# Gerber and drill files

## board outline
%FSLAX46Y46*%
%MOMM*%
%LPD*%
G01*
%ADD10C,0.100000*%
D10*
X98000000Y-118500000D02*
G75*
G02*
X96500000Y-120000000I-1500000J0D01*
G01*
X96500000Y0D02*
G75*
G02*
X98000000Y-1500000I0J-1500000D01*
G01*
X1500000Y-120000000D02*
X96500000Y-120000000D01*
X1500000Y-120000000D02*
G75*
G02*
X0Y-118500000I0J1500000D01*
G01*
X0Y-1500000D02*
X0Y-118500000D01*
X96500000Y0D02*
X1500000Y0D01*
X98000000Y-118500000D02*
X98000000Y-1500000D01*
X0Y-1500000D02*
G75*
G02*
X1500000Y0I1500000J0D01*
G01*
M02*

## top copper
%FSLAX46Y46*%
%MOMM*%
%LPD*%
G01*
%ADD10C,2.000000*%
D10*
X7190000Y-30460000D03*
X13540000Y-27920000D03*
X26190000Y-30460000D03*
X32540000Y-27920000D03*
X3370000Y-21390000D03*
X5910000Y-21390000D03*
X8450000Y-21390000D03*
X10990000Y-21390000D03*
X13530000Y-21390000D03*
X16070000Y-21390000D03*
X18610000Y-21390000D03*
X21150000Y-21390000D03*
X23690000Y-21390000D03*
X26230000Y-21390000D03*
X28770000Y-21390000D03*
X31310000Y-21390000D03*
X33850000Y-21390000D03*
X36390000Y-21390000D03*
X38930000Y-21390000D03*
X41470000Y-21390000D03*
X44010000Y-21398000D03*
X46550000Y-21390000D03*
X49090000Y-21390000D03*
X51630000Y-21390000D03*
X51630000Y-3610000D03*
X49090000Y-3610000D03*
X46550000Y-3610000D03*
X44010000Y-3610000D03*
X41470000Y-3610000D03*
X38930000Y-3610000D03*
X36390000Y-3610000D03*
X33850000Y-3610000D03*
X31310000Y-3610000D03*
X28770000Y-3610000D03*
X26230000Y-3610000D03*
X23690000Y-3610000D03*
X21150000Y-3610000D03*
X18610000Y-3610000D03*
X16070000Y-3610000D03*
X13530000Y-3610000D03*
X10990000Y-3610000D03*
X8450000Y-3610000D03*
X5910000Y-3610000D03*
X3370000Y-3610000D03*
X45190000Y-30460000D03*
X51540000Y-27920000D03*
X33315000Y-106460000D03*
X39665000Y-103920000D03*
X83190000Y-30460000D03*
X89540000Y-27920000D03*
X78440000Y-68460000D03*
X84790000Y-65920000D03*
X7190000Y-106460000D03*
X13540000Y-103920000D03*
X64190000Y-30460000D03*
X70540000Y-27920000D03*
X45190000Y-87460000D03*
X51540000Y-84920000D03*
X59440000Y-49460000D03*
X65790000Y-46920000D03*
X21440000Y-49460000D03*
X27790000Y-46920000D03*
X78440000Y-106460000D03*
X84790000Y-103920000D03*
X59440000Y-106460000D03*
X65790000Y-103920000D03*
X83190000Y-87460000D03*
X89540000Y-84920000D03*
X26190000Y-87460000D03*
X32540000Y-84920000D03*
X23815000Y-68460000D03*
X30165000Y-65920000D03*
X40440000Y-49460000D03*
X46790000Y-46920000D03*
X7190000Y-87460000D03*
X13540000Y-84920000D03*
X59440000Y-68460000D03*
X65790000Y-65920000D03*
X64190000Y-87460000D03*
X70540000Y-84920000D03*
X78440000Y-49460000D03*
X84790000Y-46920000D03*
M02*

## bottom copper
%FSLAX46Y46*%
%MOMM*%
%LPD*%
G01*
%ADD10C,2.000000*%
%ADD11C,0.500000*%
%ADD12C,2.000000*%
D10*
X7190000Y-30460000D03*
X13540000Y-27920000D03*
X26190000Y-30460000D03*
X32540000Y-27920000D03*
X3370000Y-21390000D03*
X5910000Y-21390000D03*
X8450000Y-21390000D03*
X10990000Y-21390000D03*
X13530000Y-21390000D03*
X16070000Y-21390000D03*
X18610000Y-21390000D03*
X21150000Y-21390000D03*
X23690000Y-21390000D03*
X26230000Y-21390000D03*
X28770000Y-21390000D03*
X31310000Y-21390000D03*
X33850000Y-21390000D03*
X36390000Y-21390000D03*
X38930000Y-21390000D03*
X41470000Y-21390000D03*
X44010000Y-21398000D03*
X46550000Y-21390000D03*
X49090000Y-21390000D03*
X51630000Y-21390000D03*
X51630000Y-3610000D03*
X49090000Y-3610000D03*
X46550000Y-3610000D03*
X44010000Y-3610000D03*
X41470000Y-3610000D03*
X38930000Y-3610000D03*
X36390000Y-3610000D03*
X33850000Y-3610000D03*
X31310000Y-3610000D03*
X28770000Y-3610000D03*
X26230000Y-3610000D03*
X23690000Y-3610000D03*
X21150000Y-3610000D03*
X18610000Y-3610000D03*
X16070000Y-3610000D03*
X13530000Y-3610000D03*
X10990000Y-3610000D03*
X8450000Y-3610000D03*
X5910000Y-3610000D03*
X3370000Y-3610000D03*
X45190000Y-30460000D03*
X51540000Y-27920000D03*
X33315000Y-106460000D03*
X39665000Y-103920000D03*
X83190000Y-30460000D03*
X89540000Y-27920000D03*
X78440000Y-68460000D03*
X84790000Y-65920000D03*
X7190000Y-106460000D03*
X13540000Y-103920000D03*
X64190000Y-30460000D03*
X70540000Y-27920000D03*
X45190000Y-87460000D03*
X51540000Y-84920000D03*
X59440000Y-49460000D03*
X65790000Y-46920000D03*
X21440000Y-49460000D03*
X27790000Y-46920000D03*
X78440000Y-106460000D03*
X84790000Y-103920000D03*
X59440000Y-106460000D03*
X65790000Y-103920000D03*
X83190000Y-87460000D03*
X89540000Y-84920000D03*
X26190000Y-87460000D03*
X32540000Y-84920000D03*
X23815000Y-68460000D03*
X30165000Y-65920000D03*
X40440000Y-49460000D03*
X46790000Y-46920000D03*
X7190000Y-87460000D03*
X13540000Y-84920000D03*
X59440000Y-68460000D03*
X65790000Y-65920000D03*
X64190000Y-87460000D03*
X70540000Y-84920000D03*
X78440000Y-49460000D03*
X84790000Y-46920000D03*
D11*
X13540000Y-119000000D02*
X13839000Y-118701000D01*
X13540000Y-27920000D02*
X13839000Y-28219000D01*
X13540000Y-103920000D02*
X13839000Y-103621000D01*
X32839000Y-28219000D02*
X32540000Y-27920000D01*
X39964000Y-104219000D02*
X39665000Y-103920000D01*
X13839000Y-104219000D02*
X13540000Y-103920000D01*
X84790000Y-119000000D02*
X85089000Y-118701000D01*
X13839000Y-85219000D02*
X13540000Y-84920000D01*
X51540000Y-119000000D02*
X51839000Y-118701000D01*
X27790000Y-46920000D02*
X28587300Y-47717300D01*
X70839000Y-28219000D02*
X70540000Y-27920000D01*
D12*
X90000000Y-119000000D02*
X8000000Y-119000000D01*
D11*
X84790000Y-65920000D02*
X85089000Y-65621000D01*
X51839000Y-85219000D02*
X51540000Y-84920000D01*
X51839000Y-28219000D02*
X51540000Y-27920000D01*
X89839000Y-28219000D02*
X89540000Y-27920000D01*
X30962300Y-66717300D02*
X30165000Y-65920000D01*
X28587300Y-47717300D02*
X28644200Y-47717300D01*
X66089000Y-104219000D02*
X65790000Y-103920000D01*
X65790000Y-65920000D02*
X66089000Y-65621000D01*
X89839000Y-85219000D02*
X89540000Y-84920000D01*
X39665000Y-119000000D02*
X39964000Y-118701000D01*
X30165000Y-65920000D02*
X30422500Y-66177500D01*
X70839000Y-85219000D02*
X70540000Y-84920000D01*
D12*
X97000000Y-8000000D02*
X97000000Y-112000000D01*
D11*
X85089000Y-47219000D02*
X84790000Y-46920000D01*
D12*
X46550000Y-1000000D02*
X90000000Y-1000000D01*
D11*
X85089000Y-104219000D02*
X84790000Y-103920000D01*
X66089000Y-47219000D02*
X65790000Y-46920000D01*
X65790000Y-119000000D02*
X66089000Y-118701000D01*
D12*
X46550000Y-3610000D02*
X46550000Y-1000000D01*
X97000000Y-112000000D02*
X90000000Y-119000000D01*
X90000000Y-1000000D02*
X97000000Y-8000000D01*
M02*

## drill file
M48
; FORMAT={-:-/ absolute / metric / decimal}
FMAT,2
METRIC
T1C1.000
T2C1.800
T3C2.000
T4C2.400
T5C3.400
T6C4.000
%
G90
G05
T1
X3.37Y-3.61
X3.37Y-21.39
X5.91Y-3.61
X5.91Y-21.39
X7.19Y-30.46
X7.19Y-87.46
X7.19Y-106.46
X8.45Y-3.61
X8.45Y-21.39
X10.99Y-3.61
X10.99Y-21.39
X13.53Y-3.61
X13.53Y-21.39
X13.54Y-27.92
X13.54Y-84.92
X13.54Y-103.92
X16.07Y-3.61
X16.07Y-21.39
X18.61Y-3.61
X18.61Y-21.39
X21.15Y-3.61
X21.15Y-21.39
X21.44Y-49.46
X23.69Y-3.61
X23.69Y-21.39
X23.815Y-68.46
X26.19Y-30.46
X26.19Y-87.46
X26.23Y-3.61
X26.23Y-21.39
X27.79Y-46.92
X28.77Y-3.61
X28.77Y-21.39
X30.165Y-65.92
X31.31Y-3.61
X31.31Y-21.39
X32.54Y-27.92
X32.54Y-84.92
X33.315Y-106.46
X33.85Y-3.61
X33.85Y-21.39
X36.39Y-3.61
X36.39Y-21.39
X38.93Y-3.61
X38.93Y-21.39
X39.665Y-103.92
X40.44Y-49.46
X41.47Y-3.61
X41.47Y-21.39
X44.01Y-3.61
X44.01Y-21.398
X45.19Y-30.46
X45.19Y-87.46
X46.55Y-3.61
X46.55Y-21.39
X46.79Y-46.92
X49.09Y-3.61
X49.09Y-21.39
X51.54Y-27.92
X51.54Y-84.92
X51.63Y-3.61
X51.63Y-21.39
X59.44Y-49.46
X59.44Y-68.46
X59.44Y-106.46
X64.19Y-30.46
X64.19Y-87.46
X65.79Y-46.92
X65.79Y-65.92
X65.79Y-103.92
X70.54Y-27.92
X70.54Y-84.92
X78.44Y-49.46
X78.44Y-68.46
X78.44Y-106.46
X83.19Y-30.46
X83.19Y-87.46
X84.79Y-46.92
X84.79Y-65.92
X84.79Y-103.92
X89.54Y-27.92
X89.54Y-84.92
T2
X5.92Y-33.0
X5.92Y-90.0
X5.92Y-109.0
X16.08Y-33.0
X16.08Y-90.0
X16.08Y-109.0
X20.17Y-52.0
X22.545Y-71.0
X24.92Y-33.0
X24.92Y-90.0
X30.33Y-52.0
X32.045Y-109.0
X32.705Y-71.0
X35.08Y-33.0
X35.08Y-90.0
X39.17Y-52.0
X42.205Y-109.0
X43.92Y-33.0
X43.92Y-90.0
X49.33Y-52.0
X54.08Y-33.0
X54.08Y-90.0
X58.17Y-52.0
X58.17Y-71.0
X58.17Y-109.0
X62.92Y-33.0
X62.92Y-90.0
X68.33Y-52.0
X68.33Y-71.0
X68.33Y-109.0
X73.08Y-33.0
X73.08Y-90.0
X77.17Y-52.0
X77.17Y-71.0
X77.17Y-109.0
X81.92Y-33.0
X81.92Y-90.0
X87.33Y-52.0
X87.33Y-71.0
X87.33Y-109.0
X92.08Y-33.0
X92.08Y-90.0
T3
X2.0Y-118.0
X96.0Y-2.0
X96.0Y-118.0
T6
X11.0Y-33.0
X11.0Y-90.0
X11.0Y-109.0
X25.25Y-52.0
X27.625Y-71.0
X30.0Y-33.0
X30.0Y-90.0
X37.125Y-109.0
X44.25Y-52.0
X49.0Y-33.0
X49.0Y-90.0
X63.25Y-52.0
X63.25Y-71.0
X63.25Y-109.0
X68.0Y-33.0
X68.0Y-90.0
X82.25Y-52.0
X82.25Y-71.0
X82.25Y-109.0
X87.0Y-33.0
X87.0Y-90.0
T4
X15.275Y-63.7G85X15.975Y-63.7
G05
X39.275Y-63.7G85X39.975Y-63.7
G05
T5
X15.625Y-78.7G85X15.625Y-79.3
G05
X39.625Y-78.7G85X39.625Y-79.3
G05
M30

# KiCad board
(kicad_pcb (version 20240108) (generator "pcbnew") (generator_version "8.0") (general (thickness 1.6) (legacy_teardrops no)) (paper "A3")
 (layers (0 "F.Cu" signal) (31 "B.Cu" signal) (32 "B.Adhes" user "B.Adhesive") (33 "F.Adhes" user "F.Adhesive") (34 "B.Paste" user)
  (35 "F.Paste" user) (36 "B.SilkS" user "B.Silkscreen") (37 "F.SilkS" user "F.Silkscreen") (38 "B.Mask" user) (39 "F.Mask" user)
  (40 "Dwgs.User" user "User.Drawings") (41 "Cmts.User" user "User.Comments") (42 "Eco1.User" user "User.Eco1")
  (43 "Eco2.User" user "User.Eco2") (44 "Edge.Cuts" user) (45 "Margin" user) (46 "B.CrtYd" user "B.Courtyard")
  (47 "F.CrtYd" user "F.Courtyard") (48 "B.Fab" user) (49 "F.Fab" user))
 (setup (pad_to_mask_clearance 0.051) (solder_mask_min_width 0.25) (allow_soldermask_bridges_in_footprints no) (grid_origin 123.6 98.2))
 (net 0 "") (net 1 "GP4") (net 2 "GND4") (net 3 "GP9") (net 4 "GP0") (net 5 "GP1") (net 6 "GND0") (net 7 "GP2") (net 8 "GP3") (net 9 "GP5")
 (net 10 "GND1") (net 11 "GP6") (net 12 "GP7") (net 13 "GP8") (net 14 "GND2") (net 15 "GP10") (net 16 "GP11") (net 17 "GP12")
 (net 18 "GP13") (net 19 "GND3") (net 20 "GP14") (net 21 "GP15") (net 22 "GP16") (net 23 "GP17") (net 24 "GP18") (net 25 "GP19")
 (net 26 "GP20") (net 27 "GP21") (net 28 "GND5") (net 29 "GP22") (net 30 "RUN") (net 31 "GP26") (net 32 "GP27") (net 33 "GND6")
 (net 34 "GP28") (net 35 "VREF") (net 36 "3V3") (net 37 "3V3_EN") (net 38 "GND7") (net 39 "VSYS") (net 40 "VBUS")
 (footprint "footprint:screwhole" (layer "F.Cu") (at 96 2)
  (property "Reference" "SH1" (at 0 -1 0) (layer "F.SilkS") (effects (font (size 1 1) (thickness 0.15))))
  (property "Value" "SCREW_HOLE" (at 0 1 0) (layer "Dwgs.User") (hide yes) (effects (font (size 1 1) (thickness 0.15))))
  (pad "" np_thru_hole circle (at 0 0) (size 2 2) (drill 2) (layers "*.Cu" "*.Mask")))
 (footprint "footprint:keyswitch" (layer "F.Cu") (at 11 33)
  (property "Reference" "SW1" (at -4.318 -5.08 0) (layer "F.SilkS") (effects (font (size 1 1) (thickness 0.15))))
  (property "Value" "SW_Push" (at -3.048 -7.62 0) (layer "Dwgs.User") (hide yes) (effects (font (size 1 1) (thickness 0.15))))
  (pad "" np_thru_hole circle (at -5.08 0) (size 1.8 1.8) (drill 1.8) (layers "*.Cu" "*.Mask"))
  (pad "" np_thru_hole circle (at 0 0) (size 4 4) (drill 4) (layers "*.Cu" "*.Mask"))
  (pad "" np_thru_hole circle (at 5.08 0) (size 1.8 1.8) (drill 1.8) (layers "*.Cu" "*.Mask"))
  (pad "1" thru_hole circle (at -3.81 -2.54) (size 2 2) (drill 1) (layers "*.Cu" "*.Mask") (remove_unused_layers no) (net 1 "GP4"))
  (pad "2" thru_hole circle (at 2.54 -5.08) (size 2 2) (drill 1) (layers "*.Cu" "*.Mask") (remove_unused_layers no) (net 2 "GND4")))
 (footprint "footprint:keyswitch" (layer "F.Cu") (at 30 33)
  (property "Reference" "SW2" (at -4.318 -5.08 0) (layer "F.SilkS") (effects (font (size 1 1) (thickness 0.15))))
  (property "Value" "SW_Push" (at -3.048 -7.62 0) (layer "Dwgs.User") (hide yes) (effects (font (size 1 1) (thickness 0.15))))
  (pad "" np_thru_hole circle (at -5.08 0) (size 1.8 1.8) (drill 1.8) (layers "*.Cu" "*.Mask"))
  (pad "" np_thru_hole circle (at 0 0) (size 4 4) (drill 4) (layers "*.Cu" "*.Mask"))
  (pad "" np_thru_hole circle (at 5.08 0) (size 1.8 1.8) (drill 1.8) (layers "*.Cu" "*.Mask"))
  (pad "1" thru_hole circle (at -3.81 -2.54) (size 2 2) (drill 1) (layers "*.Cu" "*.Mask") (remove_unused_layers no) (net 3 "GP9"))
  (pad "2" thru_hole circle (at 2.54 -5.08) (size 2 2) (drill 1) (layers "*.Cu" "*.Mask") (remove_unused_layers no) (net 2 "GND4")))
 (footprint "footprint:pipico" (layer "F.Cu") (at 27.5 12.5)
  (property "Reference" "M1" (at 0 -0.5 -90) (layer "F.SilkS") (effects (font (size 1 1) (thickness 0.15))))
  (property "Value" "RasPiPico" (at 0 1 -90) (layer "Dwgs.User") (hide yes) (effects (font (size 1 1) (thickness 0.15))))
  (pad "1" thru_hole circle (at -24.13 8.89 270) (size 2 2) (drill 1) (layers "*.Cu" "*.Mask") (remove_unused_layers no) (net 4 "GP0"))
  (pad "2" thru_hole circle (at -21.59 8.89 270) (size 2 2) (drill 1) (layers "*.Cu" "*.Mask") (remove_unused_layers no) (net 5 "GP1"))
  (pad "3" thru_hole circle (at -19.05 8.89 270) (size 2 2) (drill 1) (layers "*.Cu" "*.Mask") (remove_unused_layers no) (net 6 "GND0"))
  (pad "4" thru_hole circle (at -16.51 8.89 270) (size 2 2) (drill 1) (layers "*.Cu" "*.Mask") (remove_unused_layers no) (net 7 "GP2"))
  (pad "5" thru_hole circle (at -13.97 8.89 270) (size 2 2) (drill 1) (layers "*.Cu" "*.Mask") (remove_unused_layers no) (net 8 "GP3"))
  (pad "6" thru_hole circle (at -11.43 8.89 270) (size 2 2) (drill 1) (layers "*.Cu" "*.Mask") (remove_unused_layers no) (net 1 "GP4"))
  (pad "7" thru_hole circle (at -8.89 8.89 270) (size 2 2) (drill 1) (layers "*.Cu" "*.Mask") (remove_unused_layers no) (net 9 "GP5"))
  (pad "8" thru_hole circle (at -6.35 8.89 270) (size 2 2) (drill 1) (layers "*.Cu" "*.Mask") (remove_unused_layers no) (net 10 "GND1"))
  (pad "9" thru_hole circle (at -3.81 8.89 270) (size 2 2) (drill 1) (layers "*.Cu" "*.Mask") (remove_unused_layers no) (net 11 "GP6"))
  (pad "10" thru_hole circle (at -1.27 8.89 270) (size 2 2) (drill 1) (layers "*.Cu" "*.Mask") (remove_unused_layers no) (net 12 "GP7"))
  (pad "11" thru_hole circle (at 1.27 8.89 270) (size 2 2) (drill 1) (layers "*.Cu" "*.Mask") (remove_unused_layers no) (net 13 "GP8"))
  (pad "12" thru_hole circle (at 3.81 8.89 270) (size 2 2) (drill 1) (layers "*.Cu" "*.Mask") (remove_unused_layers no) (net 3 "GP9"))
  (pad "13" thru_hole circle (at 6.35 8.89 270) (size 2 2) (drill 1) (layers "*.Cu" "*.Mask") (remove_unused_layers no) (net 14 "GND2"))
  (pad "14" thru_hole circle (at 8.89 8.89 270) (size 2 2) (drill 1) (layers "*.Cu" "*.Mask") (remove_unused_layers no) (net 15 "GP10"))
  (pad "15" thru_hole circle (at 11.43 8.89 270) (size 2 2) (drill 1) (layers "*.Cu" "*.Mask") (remove_unused_layers no) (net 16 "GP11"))
  (pad "16" thru_hole circle (at 13.97 8.89 270) (size 2 2) (drill 1) (layers "*.Cu" "*.Mask") (remove_unused_layers no) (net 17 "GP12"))
  (pad "17" thru_hole circle (at 16.51 8.898 270) (size 2 2) (drill 1) (layers "*.Cu" "*.Mask") (remove_unused_layers no) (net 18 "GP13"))
  (pad "18" thru_hole circle (at 19.05 8.89 270) (size 2 2) (drill 1) (layers "*.Cu" "*.Mask") (remove_unused_layers no) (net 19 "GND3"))
  (pad "19" thru_hole circle (at 21.59 8.89 270) (size 2 2) (drill 1) (layers "*.Cu" "*.Mask") (remove_unused_layers no) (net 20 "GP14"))
  (pad "20" thru_hole circle (at 24.13 8.89 270) (size 2 2) (drill 1) (layers "*.Cu" "*.Mask") (remove_unused_layers no) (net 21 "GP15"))
  (pad "21" thru_hole circle (at 24.13 -8.89 270) (size 2 2) (drill 1) (layers "*.Cu" "*.Mask") (remove_unused_layers no) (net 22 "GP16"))
  (pad "22" thru_hole circle (at 21.59 -8.89 270) (size 2 2) (drill 1) (layers "*.Cu" "*.Mask") (remove_unused_layers no) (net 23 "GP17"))
  (pad "23" thru_hole circle (at 19.05 -8.89 270) (size 2 2) (drill 1) (layers "*.Cu" "*.Mask") (remove_unused_layers no) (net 2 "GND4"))
  (pad "24" thru_hole circle (at 16.51 -8.89 270) (size 2 2) (drill 1) (layers "*.Cu" "*.Mask") (remove_unused_layers no) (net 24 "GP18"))
  (pad "25" thru_hole circle (at 13.97 -8.89 270) (size 2 2) (drill 1) (layers "*.Cu" "*.Mask") (remove_unused_layers no) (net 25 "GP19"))
  (pad "26" thru_hole circle (at 11.43 -8.89 270) (size 2 2) (drill 1) (layers "*.Cu" "*.Mask") (remove_unused_layers no) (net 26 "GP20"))
  (pad "27" thru_hole circle (at 8.89 -8.89 270) (size 2 2) (drill 1) (layers "*.Cu" "*.Mask") (remove_unused_layers no) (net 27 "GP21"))
  (pad "28" thru_hole circle (at 6.35 -8.89 270) (size 2 2) (drill 1) (layers "*.Cu" "*.Mask") (remove_unused_layers no) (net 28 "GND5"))
  (pad "29" thru_hole circle (at 3.81 -8.89 270) (size 2 2) (drill 1) (layers "*.Cu" "*.Mask") (remove_unused_layers no) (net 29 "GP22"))
  (pad "30" thru_hole circle (at 1.27 -8.89 270) (size 2 2) (drill 1) (layers "*.Cu" "*.Mask") (remove_unused_layers no) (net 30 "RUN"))
  (pad "31" thru_hole circle (at -1.27 -8.89 270) (size 2 2) (drill 1) (layers "*.Cu" "*.Mask") (remove_unused_layers no) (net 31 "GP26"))
  (pad "32" thru_hole circle (at -3.81 -8.89 270) (size 2 2) (drill 1) (layers "*.Cu" "*.Mask") (remove_unused_layers no) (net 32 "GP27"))
  (pad "33" thru_hole circle (at -6.35 -8.89 270) (size 2 2) (drill 1) (layers "*.Cu" "*.Mask") (remove_unused_layers no) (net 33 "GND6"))
  (pad "34" thru_hole circle (at -8.89 -8.89 270) (size 2 2) (drill 1) (layers "*.Cu" "*.Mask") (remove_unused_layers no) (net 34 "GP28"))
  (pad "35" thru_hole circle (at -11.43 -8.89 270) (size 2 2) (drill 1) (layers "*.Cu" "*.Mask") (remove_unused_layers no) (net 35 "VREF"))
  (pad "36" thru_hole circle (at -13.97 -8.89 270) (size 2 2) (drill 1) (layers "*.Cu" "*.Mask") (remove_unused_layers no) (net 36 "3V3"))
  (pad "37" thru_hole circle (at -16.51 -8.89 270) (size 2 2) (drill 1) (layers "*.Cu" "*.Mask") (remove_unused_layers no) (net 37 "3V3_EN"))
  (pad "38" thru_hole circle (at -19.05 -8.89 270) (size 2 2) (drill 1) (layers "*.Cu" "*.Mask") (remove_unused_layers no) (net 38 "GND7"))
  (pad "39" thru_hole circle (at -21.59 -8.89 270) (size 2 2) (drill 1) (layers "*.Cu" "*.Mask") (remove_unused_layers no) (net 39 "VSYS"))
  (pad "40" thru_hole circle (at -24.13 -8.89 270) (size 2 2) (drill 1) (layers "*.Cu" "*.Mask") (remove_unused_layers no) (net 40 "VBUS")))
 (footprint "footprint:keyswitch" (layer "F.Cu") (at 49 33)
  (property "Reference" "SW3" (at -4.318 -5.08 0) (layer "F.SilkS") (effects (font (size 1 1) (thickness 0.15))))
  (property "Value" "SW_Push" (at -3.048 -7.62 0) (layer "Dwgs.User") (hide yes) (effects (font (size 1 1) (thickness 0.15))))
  (pad "" np_thru_hole circle (at -5.08 0) (size 1.8 1.8) (drill 1.8) (layers "*.Cu" "*.Mask"))
  (pad "" np_thru_hole circle (at 0 0) (size 4 4) (drill 4) (layers "*.Cu" "*.Mask"))
  (pad "" np_thru_hole circle (at 5.08 0) (size 1.8 1.8) (drill 1.8) (layers "*.Cu" "*.Mask"))
  (pad "1" thru_hole circle (at -3.81 -2.54) (size 2 2) (drill 1) (layers "*.Cu" "*.Mask") (remove_unused_layers no) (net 20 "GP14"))
  (pad "2" thru_hole circle (at 2.54 -5.08) (size 2 2) (drill 1) (layers "*.Cu" "*.Mask") (remove_unused_layers no) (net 2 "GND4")))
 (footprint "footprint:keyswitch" (layer "F.Cu") (at 37.125 109)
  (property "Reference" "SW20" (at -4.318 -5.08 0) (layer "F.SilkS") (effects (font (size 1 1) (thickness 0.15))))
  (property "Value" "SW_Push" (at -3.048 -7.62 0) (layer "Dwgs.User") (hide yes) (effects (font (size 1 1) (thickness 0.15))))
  (pad "" np_thru_hole circle (at -5.08 0) (size 1.8 1.8) (drill 1.8) (layers "*.Cu" "*.Mask"))
  (pad "" np_thru_hole circle (at 0 0) (size 4 4) (drill 4) (layers "*.Cu" "*.Mask"))
  (pad "" np_thru_hole circle (at 5.08 0) (size 1.8 1.8) (drill 1.8) (layers "*.Cu" "*.Mask"))
  (pad "1" thru_hole circle (at -3.81 -2.54) (size 2 2) (drill 1) (layers "*.Cu" "*.Mask") (remove_unused_layers no) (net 9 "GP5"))
  (pad "2" thru_hole circle (at 2.54 -5.08) (size 2 2) (drill 1) (layers "*.Cu" "*.Mask") (remove_unused_layers no) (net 2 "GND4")))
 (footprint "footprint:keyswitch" (layer "F.Cu") (at 87 33)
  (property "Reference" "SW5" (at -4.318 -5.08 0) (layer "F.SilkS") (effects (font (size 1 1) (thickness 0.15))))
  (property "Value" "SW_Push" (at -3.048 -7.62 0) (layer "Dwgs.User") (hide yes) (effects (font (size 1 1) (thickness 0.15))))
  (pad "" np_thru_hole circle (at -5.08 0) (size 1.8 1.8) (drill 1.8) (layers "*.Cu" "*.Mask"))
  (pad "" np_thru_hole circle (at 0 0) (size 4 4) (drill 4) (layers "*.Cu" "*.Mask"))
  (pad "" np_thru_hole circle (at 5.08 0) (size 1.8 1.8) (drill 1.8) (layers "*.Cu" "*.Mask"))
  (pad "1" thru_hole circle (at -3.81 -2.54) (size 2 2) (drill 1) (layers "*.Cu" "*.Mask") (remove_unused_layers no) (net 22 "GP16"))
  (pad "2" thru_hole circle (at 2.54 -5.08) (size 2 2) (drill 1) (layers "*.Cu" "*.Mask") (remove_unused_layers no) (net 2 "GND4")))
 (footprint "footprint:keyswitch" (layer "F.Cu") (at 82.25 71)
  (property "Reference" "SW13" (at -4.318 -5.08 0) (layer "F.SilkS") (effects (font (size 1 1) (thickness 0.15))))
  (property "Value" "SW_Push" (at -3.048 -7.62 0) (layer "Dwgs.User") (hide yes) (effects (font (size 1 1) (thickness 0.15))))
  (pad "" np_thru_hole circle (at -5.08 0) (size 1.8 1.8) (drill 1.8) (layers "*.Cu" "*.Mask"))
  (pad "" np_thru_hole circle (at 0 0) (size 4 4) (drill 4) (layers "*.Cu" "*.Mask"))
  (pad "" np_thru_hole circle (at 5.08 0) (size 1.8 1.8) (drill 1.8) (layers "*.Cu" "*.Mask"))
  (pad "1" thru_hole circle (at -3.81 -2.54) (size 2 2) (drill 1) (layers "*.Cu" "*.Mask") (remove_unused_layers no) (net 24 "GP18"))
  (pad "2" thru_hole circle (at 2.54 -5.08) (size 2 2) (drill 1) (layers "*.Cu" "*.Mask") (remove_unused_layers no) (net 2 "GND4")))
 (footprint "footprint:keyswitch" (layer "F.Cu") (at 11 109)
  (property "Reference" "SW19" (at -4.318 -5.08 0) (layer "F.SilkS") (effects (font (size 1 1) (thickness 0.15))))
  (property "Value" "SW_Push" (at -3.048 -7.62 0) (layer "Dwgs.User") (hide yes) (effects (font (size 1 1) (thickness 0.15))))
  (pad "" np_thru_hole circle (at -5.08 0) (size 1.8 1.8) (drill 1.8) (layers "*.Cu" "*.Mask"))
  (pad "" np_thru_hole circle (at 0 0) (size 4 4) (drill 4) (layers "*.Cu" "*.Mask"))
  (pad "" np_thru_hole circle (at 5.08 0) (size 1.8 1.8) (drill 1.8) (layers "*.Cu" "*.Mask"))
  (pad "1" thru_hole circle (at -3.81 -2.54) (size 2 2) (drill 1) (layers "*.Cu" "*.Mask") (remove_unused_layers no) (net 4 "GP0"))
  (pad "2" thru_hole circle (at 2.54 -5.08) (size 2 2) (drill 1) (layers "*.Cu" "*.Mask") (remove_unused_layers no) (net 2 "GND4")))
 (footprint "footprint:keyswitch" (layer "F.Cu") (at 68 33)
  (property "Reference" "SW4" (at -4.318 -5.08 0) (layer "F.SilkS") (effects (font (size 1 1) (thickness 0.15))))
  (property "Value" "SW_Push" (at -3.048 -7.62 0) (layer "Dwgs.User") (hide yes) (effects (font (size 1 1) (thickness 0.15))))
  (pad "" np_thru_hole circle (at -5.08 0) (size 1.8 1.8) (drill 1.8) (layers "*.Cu" "*.Mask"))
  (pad "" np_thru_hole circle (at 0 0) (size 4 4) (drill 4) (layers "*.Cu" "*.Mask"))
  (pad "" np_thru_hole circle (at 5.08 0) (size 1.8 1.8) (drill 1.8) (layers "*.Cu" "*.Mask"))
  (pad "1" thru_hole circle (at -3.81 -2.54) (size 2 2) (drill 1) (layers "*.Cu" "*.Mask") (remove_unused_layers no) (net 27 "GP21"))
  (pad "2" thru_hole circle (at 2.54 -5.08) (size 2 2) (drill 1) (layers "*.Cu" "*.Mask") (remove_unused_layers no) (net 2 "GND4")))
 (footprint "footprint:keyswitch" (layer "F.Cu") (at 49 90)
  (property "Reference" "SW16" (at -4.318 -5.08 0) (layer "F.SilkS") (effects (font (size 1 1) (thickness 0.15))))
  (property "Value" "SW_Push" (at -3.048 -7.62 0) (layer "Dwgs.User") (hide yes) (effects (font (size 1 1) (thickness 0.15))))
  (pad "" np_thru_hole circle (at -5.08 0) (size 1.8 1.8) (drill 1.8) (layers "*.Cu" "*.Mask"))
  (pad "" np_thru_hole circle (at 0 0) (size 4 4) (drill 4) (layers "*.Cu" "*.Mask"))
  (pad "" np_thru_hole circle (at 5.08 0) (size 1.8 1.8) (drill 1.8) (layers "*.Cu" "*.Mask"))
  (pad "1" thru_hole circle (at -3.81 -2.54) (size 2 2) (drill 1) (layers "*.Cu" "*.Mask") (remove_unused_layers no) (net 16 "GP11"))
  (pad "2" thru_hole circle (at 2.54 -5.08) (size 2 2) (drill 1) (layers "*.Cu" "*.Mask") (remove_unused_layers no) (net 2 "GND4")))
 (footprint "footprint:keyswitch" (layer "F.Cu") (at 63.25 52)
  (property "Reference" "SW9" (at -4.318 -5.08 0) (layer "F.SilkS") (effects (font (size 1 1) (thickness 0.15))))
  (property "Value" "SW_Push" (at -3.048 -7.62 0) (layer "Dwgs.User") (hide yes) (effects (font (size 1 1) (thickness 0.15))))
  (pad "" np_thru_hole circle (at -5.08 0) (size 1.8 1.8) (drill 1.8) (layers "*.Cu" "*.Mask"))
  (pad "" np_thru_hole circle (at 0 0) (size 4 4) (drill 4) (layers "*.Cu" "*.Mask"))
  (pad "" np_thru_hole circle (at 5.08 0) (size 1.8 1.8) (drill 1.8) (layers "*.Cu" "*.Mask"))
  (pad "1" thru_hole circle (at -3.81 -2.54) (size 2 2) (drill 1) (layers "*.Cu" "*.Mask") (remove_unused_layers no) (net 29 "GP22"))
  (pad "2" thru_hole circle (at 2.54 -5.08) (size 2 2) (drill 1) (layers "*.Cu" "*.Mask") (remove_unused_layers no) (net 2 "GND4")))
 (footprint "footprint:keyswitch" (layer "F.Cu") (at 25.25 52)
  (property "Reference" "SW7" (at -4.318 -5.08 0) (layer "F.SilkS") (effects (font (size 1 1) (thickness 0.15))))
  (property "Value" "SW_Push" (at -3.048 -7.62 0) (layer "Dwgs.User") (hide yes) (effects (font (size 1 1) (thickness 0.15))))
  (pad "" np_thru_hole circle (at -5.08 0) (size 1.8 1.8) (drill 1.8) (layers "*.Cu" "*.Mask"))
  (pad "" np_thru_hole circle (at 0 0) (size 4 4) (drill 4) (layers "*.Cu" "*.Mask"))
  (pad "" np_thru_hole circle (at 5.08 0) (size 1.8 1.8) (drill 1.8) (layers "*.Cu" "*.Mask"))
  (pad "1" thru_hole circle (at -3.81 -2.54) (size 2 2) (drill 1) (layers "*.Cu" "*.Mask") (remove_unused_layers no) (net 13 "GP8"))
  (pad "2" thru_hole circle (at 2.54 -5.08) (size 2 2) (drill 1) (layers "*.Cu" "*.Mask") (remove_unused_layers no) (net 2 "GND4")))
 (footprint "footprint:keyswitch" (layer "F.Cu") (at 82.25 109)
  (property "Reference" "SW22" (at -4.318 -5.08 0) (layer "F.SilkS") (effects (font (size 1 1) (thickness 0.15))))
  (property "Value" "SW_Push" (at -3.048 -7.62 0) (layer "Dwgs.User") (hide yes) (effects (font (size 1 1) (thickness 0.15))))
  (pad "" np_thru_hole circle (at -5.08 0) (size 1.8 1.8) (drill 1.8) (layers "*.Cu" "*.Mask"))
  (pad "" np_thru_hole circle (at 0 0) (size 4 4) (drill 4) (layers "*.Cu" "*.Mask"))
  (pad "" np_thru_hole circle (at 5.08 0) (size 1.8 1.8) (drill 1.8) (layers "*.Cu" "*.Mask"))
  (pad "1" thru_hole circle (at -3.81 -2.54) (size 2 2) (drill 1) (layers "*.Cu" "*.Mask") (remove_unused_layers no) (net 26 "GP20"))
  (pad "2" thru_hole circle (at 2.54 -5.08) (size 2 2) (drill 1) (layers "*.Cu" "*.Mask") (remove_unused_layers no) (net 2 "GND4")))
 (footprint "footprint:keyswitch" (layer "F.Cu") (at 63.25 109)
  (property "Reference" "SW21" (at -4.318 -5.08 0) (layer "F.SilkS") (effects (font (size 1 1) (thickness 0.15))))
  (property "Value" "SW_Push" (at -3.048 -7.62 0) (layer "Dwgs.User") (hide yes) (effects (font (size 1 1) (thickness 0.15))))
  (pad "" np_thru_hole circle (at -5.08 0) (size 1.8 1.8) (drill 1.8) (layers "*.Cu" "*.Mask"))
  (pad "" np_thru_hole circle (at 0 0) (size 4 4) (drill 4) (layers "*.Cu" "*.Mask"))
  (pad "" np_thru_hole circle (at 5.08 0) (size 1.8 1.8) (drill 1.8) (layers "*.Cu" "*.Mask"))
  (pad "1" thru_hole circle (at -3.81 -2.54) (size 2 2) (drill 1) (layers "*.Cu" "*.Mask") (remove_unused_layers no) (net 34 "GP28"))
  (pad "2" thru_hole circle (at 2.54 -5.08) (size 2 2) (drill 1) (layers "*.Cu" "*.Mask") (remove_unused_layers no) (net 2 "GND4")))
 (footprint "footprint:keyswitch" (layer "F.Cu") (at 87 90)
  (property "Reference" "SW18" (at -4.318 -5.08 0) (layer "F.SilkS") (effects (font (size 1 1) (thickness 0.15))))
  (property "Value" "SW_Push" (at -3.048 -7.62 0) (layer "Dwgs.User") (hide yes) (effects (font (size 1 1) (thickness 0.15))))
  (pad "" np_thru_hole circle (at -5.08 0) (size 1.8 1.8) (drill 1.8) (layers "*.Cu" "*.Mask"))
  (pad "" np_thru_hole circle (at 0 0) (size 4 4) (drill 4) (layers "*.Cu" "*.Mask"))
  (pad "" np_thru_hole circle (at 5.08 0) (size 1.8 1.8) (drill 1.8) (layers "*.Cu" "*.Mask"))
  (pad "1" thru_hole circle (at -3.81 -2.54) (size 2 2) (drill 1) (layers "*.Cu" "*.Mask") (remove_unused_layers no) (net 25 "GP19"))
  (pad "2" thru_hole circle (at 2.54 -5.08) (size 2 2) (drill 1) (layers "*.Cu" "*.Mask") (remove_unused_layers no) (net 2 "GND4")))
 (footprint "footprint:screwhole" (layer "F.Cu") (at 2 118)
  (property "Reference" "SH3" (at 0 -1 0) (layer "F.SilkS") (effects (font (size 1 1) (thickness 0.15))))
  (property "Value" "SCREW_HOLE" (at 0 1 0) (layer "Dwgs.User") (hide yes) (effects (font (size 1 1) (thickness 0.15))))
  (pad "" np_thru_hole circle (at 0 0) (size 2 2) (drill 2) (layers "*.Cu" "*.Mask")))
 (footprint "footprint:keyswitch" (layer "F.Cu") (at 30 90)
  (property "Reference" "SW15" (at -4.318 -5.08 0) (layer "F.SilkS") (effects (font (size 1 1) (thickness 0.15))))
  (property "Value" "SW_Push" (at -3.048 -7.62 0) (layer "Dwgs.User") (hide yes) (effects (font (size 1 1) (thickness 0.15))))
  (pad "" np_thru_hole circle (at -5.08 0) (size 1.8 1.8) (drill 1.8) (layers "*.Cu" "*.Mask"))
  (pad "" np_thru_hole circle (at 0 0) (size 4 4) (drill 4) (layers "*.Cu" "*.Mask"))
  (pad "" np_thru_hole circle (at 5.08 0) (size 1.8 1.8) (drill 1.8) (layers "*.Cu" "*.Mask"))
  (pad "1" thru_hole circle (at -3.81 -2.54) (size 2 2) (drill 1) (layers "*.Cu" "*.Mask") (remove_unused_layers no) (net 11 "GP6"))
  (pad "2" thru_hole circle (at 2.54 -5.08) (size 2 2) (drill 1) (layers "*.Cu" "*.Mask") (remove_unused_layers no) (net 2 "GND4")))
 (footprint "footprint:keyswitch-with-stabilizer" (layer "F.Cu") (at 27.625 71)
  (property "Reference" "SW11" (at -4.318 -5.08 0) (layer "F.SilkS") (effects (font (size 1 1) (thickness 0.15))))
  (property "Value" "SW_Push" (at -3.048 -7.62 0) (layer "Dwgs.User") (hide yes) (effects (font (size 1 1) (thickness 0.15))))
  (pad "" np_thru_hole oval (at -12 -7.3) (size 3.1 2.4) (drill oval 3.1 2.4) (layers "*.Cu" "*.Mask"))
  (pad "" np_thru_hole oval (at -12 8) (size 3.4 4) (drill oval 3.4 4) (layers "*.Cu" "*.Mask"))
  (pad "" np_thru_hole circle (at -5.08 0) (size 1.8 1.8) (drill 1.8) (layers "*.Cu" "*.Mask"))
  (pad "" np_thru_hole circle (at 0 0) (size 4 4) (drill 4) (layers "*.Cu" "*.Mask"))
  (pad "" np_thru_hole circle (at 5.08 0) (size 1.8 1.8) (drill 1.8) (layers "*.Cu" "*.Mask"))
  (pad "" np_thru_hole oval (at 12 -7.3) (size 3.1 2.4) (drill oval 3.1 2.4) (layers "*.Cu" "*.Mask"))
  (pad "" np_thru_hole oval (at 12 8) (size 3.4 4) (drill oval 3.4 4) (layers "*.Cu" "*.Mask"))
  (pad "1" thru_hole circle (at -3.81 -2.54) (size 2 2) (drill 1) (layers "*.Cu" "*.Mask") (remove_unused_layers no) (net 12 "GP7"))
  (pad "2" thru_hole circle (at 2.54 -5.08) (size 2 2) (drill 1) (layers "*.Cu" "*.Mask") (remove_unused_layers no) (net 2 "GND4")))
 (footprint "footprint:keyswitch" (layer "F.Cu") (at 44.25 52)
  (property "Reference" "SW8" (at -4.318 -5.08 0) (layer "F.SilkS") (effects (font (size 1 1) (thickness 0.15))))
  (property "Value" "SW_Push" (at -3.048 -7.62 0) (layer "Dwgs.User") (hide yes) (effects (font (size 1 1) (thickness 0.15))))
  (pad "" np_thru_hole circle (at -5.08 0) (size 1.8 1.8) (drill 1.8) (layers "*.Cu" "*.Mask"))
  (pad "" np_thru_hole circle (at 0 0) (size 4 4) (drill 4) (layers "*.Cu" "*.Mask"))
  (pad "" np_thru_hole circle (at 5.08 0) (size 1.8 1.8) (drill 1.8) (layers "*.Cu" "*.Mask"))
  (pad "1" thru_hole circle (at -3.81 -2.54) (size 2 2) (drill 1) (layers "*.Cu" "*.Mask") (remove_unused_layers no) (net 18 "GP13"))
  (pad "2" thru_hole circle (at 2.54 -5.08) (size 2 2) (drill 1) (layers "*.Cu" "*.Mask") (remove_unused_layers no) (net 2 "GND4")))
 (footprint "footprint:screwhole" (layer "F.Cu") (at 96 118)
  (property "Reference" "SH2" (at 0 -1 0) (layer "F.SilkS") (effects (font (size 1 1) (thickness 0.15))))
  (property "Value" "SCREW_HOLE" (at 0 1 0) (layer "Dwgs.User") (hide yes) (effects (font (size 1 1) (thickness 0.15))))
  (pad "" np_thru_hole circle (at 0 0) (size 2 2) (drill 2) (layers "*.Cu" "*.Mask")))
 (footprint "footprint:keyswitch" (layer "F.Cu") (at 11 90)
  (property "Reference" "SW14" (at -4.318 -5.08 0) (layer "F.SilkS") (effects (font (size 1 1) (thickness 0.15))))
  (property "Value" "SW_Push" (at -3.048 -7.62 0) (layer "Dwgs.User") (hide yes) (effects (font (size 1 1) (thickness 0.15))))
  (pad "" np_thru_hole circle (at -5.08 0) (size 1.8 1.8) (drill 1.8) (layers "*.Cu" "*.Mask"))
  (pad "" np_thru_hole circle (at 0 0) (size 4 4) (drill 4) (layers "*.Cu" "*.Mask"))
  (pad "" np_thru_hole circle (at 5.08 0) (size 1.8 1.8) (drill 1.8) (layers "*.Cu" "*.Mask"))
  (pad "1" thru_hole circle (at -3.81 -2.54) (size 2 2) (drill 1) (layers "*.Cu" "*.Mask") (remove_unused_layers no) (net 5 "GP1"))
  (pad "2" thru_hole circle (at 2.54 -5.08) (size 2 2) (drill 1) (layers "*.Cu" "*.Mask") (remove_unused_layers no) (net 2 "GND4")))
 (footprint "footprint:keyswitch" (layer "F.Cu") (at 63.25 71)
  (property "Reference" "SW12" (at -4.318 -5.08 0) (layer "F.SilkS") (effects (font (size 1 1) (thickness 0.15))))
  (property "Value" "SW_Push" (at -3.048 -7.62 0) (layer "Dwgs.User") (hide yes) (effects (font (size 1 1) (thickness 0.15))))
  (pad "" np_thru_hole circle (at -5.08 0) (size 1.8 1.8) (drill 1.8) (layers "*.Cu" "*.Mask"))
  (pad "" np_thru_hole circle (at 0 0) (size 4 4) (drill 4) (layers "*.Cu" "*.Mask"))
  (pad "" np_thru_hole circle (at 5.08 0) (size 1.8 1.8) (drill 1.8) (layers "*.Cu" "*.Mask"))
  (pad "1" thru_hole circle (at -3.81 -2.54) (size 2 2) (drill 1) (layers "*.Cu" "*.Mask") (remove_unused_layers no) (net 31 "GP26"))
  (pad "2" thru_hole circle (at 2.54 -5.08) (size 2 2) (drill 1) (layers "*.Cu" "*.Mask") (remove_unused_layers no) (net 2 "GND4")))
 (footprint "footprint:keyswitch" (layer "F.Cu") (at 68 90)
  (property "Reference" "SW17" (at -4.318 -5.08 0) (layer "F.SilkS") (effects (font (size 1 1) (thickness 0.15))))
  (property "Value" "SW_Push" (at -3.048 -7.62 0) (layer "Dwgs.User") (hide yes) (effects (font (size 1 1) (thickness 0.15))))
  (pad "" np_thru_hole circle (at -5.08 0) (size 1.8 1.8) (drill 1.8) (layers "*.Cu" "*.Mask"))
  (pad "" np_thru_hole circle (at 0 0) (size 4 4) (drill 4) (layers "*.Cu" "*.Mask"))
  (pad "" np_thru_hole circle (at 5.08 0) (size 1.8 1.8) (drill 1.8) (layers "*.Cu" "*.Mask"))
  (pad "1" thru_hole circle (at -3.81 -2.54) (size 2 2) (drill 1) (layers "*.Cu" "*.Mask") (remove_unused_layers no) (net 32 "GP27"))
  (pad "2" thru_hole circle (at 2.54 -5.08) (size 2 2) (drill 1) (layers "*.Cu" "*.Mask") (remove_unused_layers no) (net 2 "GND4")))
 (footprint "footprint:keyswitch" (layer "F.Cu") (at 82.25 52)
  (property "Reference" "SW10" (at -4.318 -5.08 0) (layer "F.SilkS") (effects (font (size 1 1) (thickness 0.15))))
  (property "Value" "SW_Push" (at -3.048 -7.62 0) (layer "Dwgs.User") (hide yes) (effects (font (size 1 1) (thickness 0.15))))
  (pad "" np_thru_hole circle (at -5.08 0) (size 1.8 1.8) (drill 1.8) (layers "*.Cu" "*.Mask"))
  (pad "" np_thru_hole circle (at 0 0) (size 4 4) (drill 4) (layers "*.Cu" "*.Mask"))
  (pad "" np_thru_hole circle (at 5.08 0) (size 1.8 1.8) (drill 1.8) (layers "*.Cu" "*.Mask"))
  (pad "1" thru_hole circle (at -3.81 -2.54) (size 2 2) (drill 1) (layers "*.Cu" "*.Mask") (remove_unused_layers no) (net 23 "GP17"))
  (pad "2" thru_hole circle (at 2.54 -5.08) (size 2 2) (drill 1) (layers "*.Cu" "*.Mask") (remove_unused_layers no) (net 2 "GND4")))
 (gr_arc (start 98 118.5) (mid 97.56066 119.56066) (end 96.5 120) (stroke (width 0.1) (type solid)) (layer "Edge.Cuts"))
 (gr_arc (start 96.5 0) (mid 97.56066 0.43934) (end 98 1.5) (stroke (width 0.1) (type solid)) (layer "Edge.Cuts"))
 (gr_line (start 1.5 120) (end 96.5 120) (stroke (width 0.1) (type solid)) (layer "Edge.Cuts"))
 (gr_arc (start 1.5 120) (mid 0.43934 119.56066) (end 0 118.5) (stroke (width 0.1) (type solid)) (layer "Edge.Cuts"))
 (gr_line (start 0 1.5) (end 0 118.5) (stroke (width 0.1) (type solid)) (layer "Edge.Cuts"))
 (gr_line (start 96.5 0) (end 1.5 0) (stroke (width 0.1) (type solid)) (layer "Edge.Cuts"))
 (gr_line (start 98 118.5) (end 98 1.5) (stroke (width 0.1) (type solid)) (layer "Edge.Cuts"))
 (gr_arc (start 0 1.5) (mid 0.43934 0.43934) (end 1.5 0) (stroke (width 0.1) (type solid)) (layer "Edge.Cuts"))
 (segment (start 13.54 119) (end 13.839 118.701) (width 0.5) (layer "B.Cu") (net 2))
 (segment (start 13.54 27.92) (end 13.839 28.219) (width 0.5) (layer "B.Cu") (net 2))
 (segment (start 13.54 103.92) (end 13.839 103.621) (width 0.5) (layer "B.Cu") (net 2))
 (segment (start 32.839 28.219) (end 32.54 27.92) (width 0.5) (layer "B.Cu") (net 2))
 (segment (start 39.964 104.219) (end 39.665 103.92) (width 0.5) (layer "B.Cu") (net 2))
 (segment (start 13.839 104.219) (end 13.54 103.92) (width 0.5) (layer "B.Cu") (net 2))
 (segment (start 84.79 119) (end 85.089 118.701) (width 0.5) (layer "B.Cu") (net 2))
 (segment (start 13.839 85.219) (end 13.54 84.92) (width 0.5) (layer "B.Cu") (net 2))
 (segment (start 51.54 119) (end 51.839 118.701) (width 0.5) (layer "B.Cu") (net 2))
 (segment (start 27.79 46.92) (end 28.5873 47.7173) (width 0.5) (layer "B.Cu") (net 2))
 (segment (start 70.839 28.219) (end 70.54 27.92) (width 0.5) (layer "B.Cu") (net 2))
 (segment (start 90 119) (end 8 119) (width 2) (layer "B.Cu") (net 2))
 (segment (start 84.79 65.92) (end 85.089 65.621) (width 0.5) (layer "B.Cu") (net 2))
 (segment (start 51.839 85.219) (end 51.54 84.92) (width 0.5) (layer "B.Cu") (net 2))
 (segment (start 51.839 28.219) (end 51.54 27.92) (width 0.5) (layer "B.Cu") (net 2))
 (segment (start 89.839 28.219) (end 89.54 27.92) (width 0.5) (layer "B.Cu") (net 2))
 (segment (start 30.9623 66.7173) (end 30.165 65.92) (width 0.5) (layer "B.Cu") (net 2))
 (segment (start 28.5873 47.7173) (end 28.6442 47.7173) (width 0.5) (layer "B.Cu") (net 2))
 (segment (start 66.089 104.219) (end 65.79 103.92) (width 0.5) (layer "B.Cu") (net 2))
 (segment (start 65.79 65.92) (end 66.089 65.621) (width 0.5) (layer "B.Cu") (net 2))
 (segment (start 89.839 85.219) (end 89.54 84.92) (width 0.5) (layer "B.Cu") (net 2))
 (segment (start 39.665 119) (end 39.964 118.701) (width 0.5) (layer "B.Cu") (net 2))
 (segment (start 30.165 65.92) (end 30.4225 66.1775) (width 0.5) (layer "B.Cu") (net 2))
 (segment (start 70.839 85.219) (end 70.54 84.92) (width 0.5) (layer "B.Cu") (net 2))
 (segment (start 97 8) (end 97 112) (width 2) (layer "B.Cu") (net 2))
 (segment (start 85.089 47.219) (end 84.79 46.92) (width 0.5) (layer "B.Cu") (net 2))
 (segment (start 46.55 1) (end 90 1) (width 2) (layer "B.Cu") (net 2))
 (segment (start 85.089 104.219) (end 84.79 103.92) (width 0.5) (layer "B.Cu") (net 2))
 (segment (start 66.089 47.219) (end 65.79 46.92) (width 0.5) (layer "B.Cu") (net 2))
 (segment (start 65.79 119) (end 66.089 118.701) (width 0.5) (layer "B.Cu") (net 2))
 (segment (start 46.55 3.61) (end 46.55 1) (width 2) (layer "B.Cu") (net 2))
 (segment (start 97 112) (end 90 119) (width 2) (layer "B.Cu") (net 2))
 (segment (start 90 1) (end 97 8) (width 2) (layer "B.Cu") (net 2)))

